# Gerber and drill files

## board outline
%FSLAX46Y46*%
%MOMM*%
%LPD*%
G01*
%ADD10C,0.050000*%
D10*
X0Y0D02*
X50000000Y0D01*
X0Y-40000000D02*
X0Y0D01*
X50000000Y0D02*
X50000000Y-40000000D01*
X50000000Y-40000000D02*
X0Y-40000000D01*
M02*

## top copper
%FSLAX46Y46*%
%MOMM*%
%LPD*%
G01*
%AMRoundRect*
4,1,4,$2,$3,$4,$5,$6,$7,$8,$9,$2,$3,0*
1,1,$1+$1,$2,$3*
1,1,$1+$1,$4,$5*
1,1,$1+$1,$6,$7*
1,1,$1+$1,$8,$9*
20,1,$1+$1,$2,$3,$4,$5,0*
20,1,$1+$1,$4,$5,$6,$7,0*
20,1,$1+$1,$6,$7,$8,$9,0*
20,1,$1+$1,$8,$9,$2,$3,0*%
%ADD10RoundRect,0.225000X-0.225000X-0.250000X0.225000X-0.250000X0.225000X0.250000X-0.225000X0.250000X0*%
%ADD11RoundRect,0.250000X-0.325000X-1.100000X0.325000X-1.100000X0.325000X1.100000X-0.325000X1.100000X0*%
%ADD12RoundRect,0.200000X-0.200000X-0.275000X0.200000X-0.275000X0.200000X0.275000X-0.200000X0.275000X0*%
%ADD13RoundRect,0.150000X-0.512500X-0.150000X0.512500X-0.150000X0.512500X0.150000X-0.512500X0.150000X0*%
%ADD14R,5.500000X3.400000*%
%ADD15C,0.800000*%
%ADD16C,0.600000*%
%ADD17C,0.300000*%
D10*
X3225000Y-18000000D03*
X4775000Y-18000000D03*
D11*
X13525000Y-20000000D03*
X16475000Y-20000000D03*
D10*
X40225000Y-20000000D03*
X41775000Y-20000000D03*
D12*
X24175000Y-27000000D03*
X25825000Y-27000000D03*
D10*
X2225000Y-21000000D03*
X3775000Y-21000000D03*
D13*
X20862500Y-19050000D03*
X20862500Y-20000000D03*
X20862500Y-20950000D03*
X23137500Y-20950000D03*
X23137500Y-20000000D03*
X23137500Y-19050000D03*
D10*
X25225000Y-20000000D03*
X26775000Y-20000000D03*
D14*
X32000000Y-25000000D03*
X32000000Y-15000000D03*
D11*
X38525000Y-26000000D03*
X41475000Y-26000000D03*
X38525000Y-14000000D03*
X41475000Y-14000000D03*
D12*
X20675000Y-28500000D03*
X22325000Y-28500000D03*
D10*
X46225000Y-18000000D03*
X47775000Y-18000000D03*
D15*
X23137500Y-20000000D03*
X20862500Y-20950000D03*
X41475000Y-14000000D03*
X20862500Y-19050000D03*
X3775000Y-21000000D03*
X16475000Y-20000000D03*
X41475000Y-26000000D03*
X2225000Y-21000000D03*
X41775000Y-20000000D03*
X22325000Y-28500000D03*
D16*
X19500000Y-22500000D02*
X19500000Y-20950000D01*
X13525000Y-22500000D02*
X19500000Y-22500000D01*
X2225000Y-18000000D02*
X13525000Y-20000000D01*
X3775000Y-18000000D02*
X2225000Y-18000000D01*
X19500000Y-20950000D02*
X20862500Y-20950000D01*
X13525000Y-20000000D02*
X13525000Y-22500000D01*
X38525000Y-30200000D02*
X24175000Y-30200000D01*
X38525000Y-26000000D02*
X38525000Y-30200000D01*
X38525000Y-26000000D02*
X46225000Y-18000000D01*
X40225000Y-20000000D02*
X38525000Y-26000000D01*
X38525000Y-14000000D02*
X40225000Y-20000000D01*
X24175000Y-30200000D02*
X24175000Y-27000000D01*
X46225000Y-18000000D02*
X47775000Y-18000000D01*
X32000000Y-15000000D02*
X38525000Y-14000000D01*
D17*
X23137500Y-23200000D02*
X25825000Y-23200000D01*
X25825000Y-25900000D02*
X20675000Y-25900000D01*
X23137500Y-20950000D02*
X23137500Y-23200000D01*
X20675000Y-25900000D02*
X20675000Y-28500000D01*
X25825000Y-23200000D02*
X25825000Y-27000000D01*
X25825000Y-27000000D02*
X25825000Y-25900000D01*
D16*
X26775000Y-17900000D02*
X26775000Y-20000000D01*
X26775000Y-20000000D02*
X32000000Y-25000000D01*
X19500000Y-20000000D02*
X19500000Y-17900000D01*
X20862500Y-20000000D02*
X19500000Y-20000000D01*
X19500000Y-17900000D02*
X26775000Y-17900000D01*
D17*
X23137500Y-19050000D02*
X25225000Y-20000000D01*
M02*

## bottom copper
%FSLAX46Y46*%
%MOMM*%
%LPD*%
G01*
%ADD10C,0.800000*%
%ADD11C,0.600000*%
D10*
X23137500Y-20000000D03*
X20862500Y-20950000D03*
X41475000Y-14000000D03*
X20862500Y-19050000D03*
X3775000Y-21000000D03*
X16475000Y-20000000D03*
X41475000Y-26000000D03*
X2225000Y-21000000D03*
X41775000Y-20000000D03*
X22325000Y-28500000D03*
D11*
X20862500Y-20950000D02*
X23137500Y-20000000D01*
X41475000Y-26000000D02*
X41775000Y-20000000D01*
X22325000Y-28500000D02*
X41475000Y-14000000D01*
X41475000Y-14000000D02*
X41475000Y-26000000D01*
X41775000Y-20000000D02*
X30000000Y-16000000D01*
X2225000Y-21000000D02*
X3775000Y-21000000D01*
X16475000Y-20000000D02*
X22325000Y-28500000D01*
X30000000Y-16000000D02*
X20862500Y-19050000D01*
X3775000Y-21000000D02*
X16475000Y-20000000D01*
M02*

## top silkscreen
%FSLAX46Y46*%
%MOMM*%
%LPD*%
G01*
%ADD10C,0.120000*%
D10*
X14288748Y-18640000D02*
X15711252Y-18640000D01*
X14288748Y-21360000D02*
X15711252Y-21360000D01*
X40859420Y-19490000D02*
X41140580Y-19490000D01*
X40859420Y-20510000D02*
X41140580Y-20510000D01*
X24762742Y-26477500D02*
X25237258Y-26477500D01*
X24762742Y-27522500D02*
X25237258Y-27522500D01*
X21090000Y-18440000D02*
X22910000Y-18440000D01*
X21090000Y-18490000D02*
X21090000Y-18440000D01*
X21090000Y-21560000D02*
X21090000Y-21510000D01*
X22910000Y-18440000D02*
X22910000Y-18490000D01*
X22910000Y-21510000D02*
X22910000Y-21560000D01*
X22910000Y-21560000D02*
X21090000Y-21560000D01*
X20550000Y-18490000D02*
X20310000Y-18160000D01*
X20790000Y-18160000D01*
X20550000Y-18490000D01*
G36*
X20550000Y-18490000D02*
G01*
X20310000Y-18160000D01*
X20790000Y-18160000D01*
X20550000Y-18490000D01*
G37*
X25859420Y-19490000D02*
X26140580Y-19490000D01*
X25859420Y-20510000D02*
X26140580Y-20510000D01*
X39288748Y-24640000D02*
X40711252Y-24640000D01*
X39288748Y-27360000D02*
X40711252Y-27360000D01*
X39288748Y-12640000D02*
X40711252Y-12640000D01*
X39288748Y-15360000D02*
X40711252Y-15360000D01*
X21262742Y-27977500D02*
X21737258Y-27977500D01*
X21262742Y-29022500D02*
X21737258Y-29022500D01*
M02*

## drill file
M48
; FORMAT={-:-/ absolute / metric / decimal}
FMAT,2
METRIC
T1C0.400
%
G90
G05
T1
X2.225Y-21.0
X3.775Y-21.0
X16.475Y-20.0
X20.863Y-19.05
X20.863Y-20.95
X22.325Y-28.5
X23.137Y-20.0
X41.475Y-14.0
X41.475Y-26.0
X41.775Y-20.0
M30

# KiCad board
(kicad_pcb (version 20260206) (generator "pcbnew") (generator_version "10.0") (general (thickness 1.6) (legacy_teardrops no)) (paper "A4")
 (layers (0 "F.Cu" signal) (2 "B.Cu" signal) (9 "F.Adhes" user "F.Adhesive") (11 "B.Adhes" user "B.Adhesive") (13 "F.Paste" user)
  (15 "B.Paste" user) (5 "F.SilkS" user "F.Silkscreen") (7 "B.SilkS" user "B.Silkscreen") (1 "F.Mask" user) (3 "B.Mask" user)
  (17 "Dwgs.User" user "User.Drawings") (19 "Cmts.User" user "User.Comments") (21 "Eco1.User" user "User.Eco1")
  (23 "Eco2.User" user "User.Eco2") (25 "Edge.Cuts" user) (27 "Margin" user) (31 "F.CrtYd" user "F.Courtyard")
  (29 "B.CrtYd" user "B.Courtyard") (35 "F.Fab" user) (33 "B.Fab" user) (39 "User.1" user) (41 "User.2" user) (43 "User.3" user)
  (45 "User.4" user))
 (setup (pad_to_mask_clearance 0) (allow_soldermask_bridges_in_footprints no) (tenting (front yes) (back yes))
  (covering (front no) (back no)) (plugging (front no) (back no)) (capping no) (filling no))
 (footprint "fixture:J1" (layer "F.Cu") (at 4 18)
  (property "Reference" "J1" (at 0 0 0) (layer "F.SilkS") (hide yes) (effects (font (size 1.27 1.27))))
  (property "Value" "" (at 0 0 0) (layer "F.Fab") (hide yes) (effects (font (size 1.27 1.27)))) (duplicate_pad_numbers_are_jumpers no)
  (pad "1" smd roundrect (at -0.775 0) (size 0.9 0.95) (layers "F.Cu" "F.Mask" "F.Paste") (roundrect_rratio 0.25) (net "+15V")
   (thermal_bridge_angle 45))
  (pad "2" smd roundrect (at 0.775 0) (size 0.9 0.95) (layers "F.Cu" "F.Mask" "F.Paste") (roundrect_rratio 0.25) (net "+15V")
   (thermal_bridge_angle 45)))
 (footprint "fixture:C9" (layer "F.Cu") (at 15 20)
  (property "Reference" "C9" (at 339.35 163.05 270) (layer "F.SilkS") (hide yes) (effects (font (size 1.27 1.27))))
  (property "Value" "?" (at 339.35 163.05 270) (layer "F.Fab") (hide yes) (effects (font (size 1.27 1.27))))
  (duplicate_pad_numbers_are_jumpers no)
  (fp_line (start -0.711252 -1.36) (end 0.711252 -1.36) (stroke (width 0.12) (type solid)) (layer "F.SilkS"))
  (fp_line (start -0.711252 1.36) (end 0.711252 1.36) (stroke (width 0.12) (type solid)) (layer "F.SilkS"))
  (pad "1" smd roundrect (at -1.475 0) (size 1.15 2.7) (layers "F.Cu" "F.Mask" "F.Paste") (roundrect_rratio 0.217391) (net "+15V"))
  (pad "2" smd roundrect (at 1.475 0) (size 1.15 2.7) (layers "F.Cu" "F.Mask" "F.Paste") (roundrect_rratio 0.217391) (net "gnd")))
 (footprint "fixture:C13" (layer "F.Cu") (at 41 20)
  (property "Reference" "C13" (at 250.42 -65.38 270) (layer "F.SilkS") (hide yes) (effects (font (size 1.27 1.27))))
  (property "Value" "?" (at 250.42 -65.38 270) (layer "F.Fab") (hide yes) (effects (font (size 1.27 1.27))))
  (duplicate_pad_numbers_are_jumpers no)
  (fp_line (start -0.14058 -0.51) (end 0.14058 -0.51) (stroke (width 0.12) (type solid)) (layer "F.SilkS"))
  (fp_line (start -0.14058 0.51) (end 0.14058 0.51) (stroke (width 0.12) (type solid)) (layer "F.SilkS"))
  (pad "1" smd roundrect (at -0.775 0) (size 0.9 0.95) (layers "F.Cu" "F.Mask" "F.Paste") (roundrect_rratio 0.25) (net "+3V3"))
  (pad "2" smd roundrect (at 0.775 0) (size 0.9 0.95) (layers "F.Cu" "F.Mask" "F.Paste") (roundrect_rratio 0.25) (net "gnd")))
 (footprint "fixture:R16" (layer "F.Cu") (at 25 27)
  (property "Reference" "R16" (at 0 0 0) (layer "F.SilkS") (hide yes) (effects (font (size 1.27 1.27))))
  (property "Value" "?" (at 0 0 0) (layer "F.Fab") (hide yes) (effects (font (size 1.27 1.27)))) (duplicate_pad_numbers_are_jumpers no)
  (fp_line (start -0.237258 -0.5225) (end 0.237258 -0.5225) (stroke (width 0.12) (type solid)) (layer "F.SilkS"))
  (fp_line (start -0.237258 0.5225) (end 0.237258 0.5225) (stroke (width 0.12) (type solid)) (layer "F.SilkS"))
  (pad "1" smd roundrect (at -0.825 0) (size 0.8 0.95) (layers "F.Cu" "F.Mask" "F.Paste") (roundrect_rratio 0.25) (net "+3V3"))
  (pad "2" smd roundrect (at 0.825 0) (size 0.8 0.95) (layers "F.Cu" "F.Mask" "F.Paste") (roundrect_rratio 0.25) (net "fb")))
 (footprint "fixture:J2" (layer "F.Cu") (at 3 21)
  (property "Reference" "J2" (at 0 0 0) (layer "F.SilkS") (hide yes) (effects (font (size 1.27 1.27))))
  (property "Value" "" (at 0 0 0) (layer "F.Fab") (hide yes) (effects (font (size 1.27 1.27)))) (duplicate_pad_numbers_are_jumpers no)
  (pad "1" smd roundrect (at -0.775 0) (size 0.9 0.95) (layers "F.Cu" "F.Mask" "F.Paste") (roundrect_rratio 0.25) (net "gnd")
   (thermal_bridge_angle 45))
  (pad "2" smd roundrect (at 0.775 0) (size 0.9 0.95) (layers "F.Cu" "F.Mask" "F.Paste") (roundrect_rratio 0.25) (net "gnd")
   (thermal_bridge_angle 45)))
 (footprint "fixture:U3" (layer "F.Cu") (at 22 20)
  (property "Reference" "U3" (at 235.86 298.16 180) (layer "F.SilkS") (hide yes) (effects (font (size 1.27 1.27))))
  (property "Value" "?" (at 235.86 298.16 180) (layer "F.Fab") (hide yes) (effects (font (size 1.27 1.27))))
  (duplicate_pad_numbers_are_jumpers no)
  (fp_line (start -0.91 -1.56) (end 0.91 -1.56) (stroke (width 0.12) (type solid)) (layer "F.SilkS"))
  (fp_line (start -0.91 -1.51) (end -0.91 -1.56) (stroke (width 0.12) (type solid)) (layer "F.SilkS"))
  (fp_line (start -0.91 1.56) (end -0.91 1.51) (stroke (width 0.12) (type solid)) (layer "F.SilkS"))
  (fp_line (start 0.91 -1.56) (end 0.91 -1.51) (stroke (width 0.12) (type solid)) (layer "F.SilkS"))
  (fp_line (start 0.91 1.51) (end 0.91 1.56) (stroke (width 0.12) (type solid)) (layer "F.SilkS"))
  (fp_line (start 0.91 1.56) (end -0.91 1.56) (stroke (width 0.12) (type solid)) (layer "F.SilkS"))
  (fp_poly (pts (xy -1.45 -1.51) (xy -1.69 -1.84) (xy -1.21 -1.84)) (stroke (width 0.12) (type solid)) (fill yes) (layer "F.SilkS"))
  (pad "1" smd roundrect (at -1.1375 -0.95) (size 1.325 0.6) (layers "F.Cu" "F.Mask" "F.Paste") (roundrect_rratio 0.25) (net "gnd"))
  (pad "2" smd roundrect (at -1.1375 0) (size 1.325 0.6) (layers "F.Cu" "F.Mask" "F.Paste") (roundrect_rratio 0.25) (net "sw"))
  (pad "3" smd roundrect (at -1.1375 0.95) (size 1.325 0.6) (layers "F.Cu" "F.Mask" "F.Paste") (roundrect_rratio 0.25) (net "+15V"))
  (pad "4" smd roundrect (at 1.1375 0.95) (size 1.325 0.6) (layers "F.Cu" "F.Mask" "F.Paste") (roundrect_rratio 0.25) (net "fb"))
  (pad "5" smd roundrect (at 1.1375 0) (size 1.325 0.6) (layers "F.Cu" "F.Mask" "F.Paste") (roundrect_rratio 0.25) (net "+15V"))
  (pad "6" smd roundrect (at 1.1375 -0.95) (size 1.325 0.6) (layers "F.Cu" "F.Mask" "F.Paste") (roundrect_rratio 0.25) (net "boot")))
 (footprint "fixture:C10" (layer "F.Cu") (at 26 20)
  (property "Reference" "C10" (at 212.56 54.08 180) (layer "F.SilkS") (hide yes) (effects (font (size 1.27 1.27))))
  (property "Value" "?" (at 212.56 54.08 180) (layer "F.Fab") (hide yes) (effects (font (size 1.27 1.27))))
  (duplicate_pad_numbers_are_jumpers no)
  (fp_line (start -0.14058 -0.51) (end 0.14058 -0.51) (stroke (width 0.12) (type solid)) (layer "F.SilkS"))
  (fp_line (start -0.14058 0.51) (end 0.14058 0.51) (stroke (width 0.12) (type solid)) (layer "F.SilkS"))
  (pad "1" smd roundrect (at -0.775 0) (size 0.9 0.95) (layers "F.Cu" "F.Mask" "F.Paste") (roundrect_rratio 0.25) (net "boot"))
  (pad "2" smd roundrect (at 0.775 0) (size 0.9 0.95) (layers "F.Cu" "F.Mask" "F.Paste") (roundrect_rratio 0.25) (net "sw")))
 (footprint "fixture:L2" (layer "F.Cu") (at 32 20 90)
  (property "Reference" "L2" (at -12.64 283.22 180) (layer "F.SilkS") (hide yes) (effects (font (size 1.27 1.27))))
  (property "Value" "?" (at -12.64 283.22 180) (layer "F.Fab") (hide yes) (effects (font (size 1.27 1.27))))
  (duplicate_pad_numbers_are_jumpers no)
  (pad "1" smd rect (at -5 0 90) (size 3.4 5.5) (layers "F.Cu" "F.Mask" "F.Paste") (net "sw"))
  (pad "2" smd rect (at 5 0 90) (size 3.4 5.5) (layers "F.Cu" "F.Mask" "F.Paste") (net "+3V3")))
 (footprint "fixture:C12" (layer "F.Cu") (at 40 26)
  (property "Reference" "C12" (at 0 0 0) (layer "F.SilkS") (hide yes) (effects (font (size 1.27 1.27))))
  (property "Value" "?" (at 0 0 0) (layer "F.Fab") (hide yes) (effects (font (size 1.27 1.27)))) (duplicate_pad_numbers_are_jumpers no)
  (fp_line (start -0.711252 -1.36) (end 0.711252 -1.36) (stroke (width 0.12) (type solid)) (layer "F.SilkS"))
  (fp_line (start -0.711252 1.36) (end 0.711252 1.36) (stroke (width 0.12) (type solid)) (layer "F.SilkS"))
  (pad "1" smd roundrect (at -1.475 0) (size 1.15 2.7) (layers "F.Cu" "F.Mask" "F.Paste") (roundrect_rratio 0.217391) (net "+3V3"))
  (pad "2" smd roundrect (at 1.475 0) (size 1.15 2.7) (layers "F.Cu" "F.Mask" "F.Paste") (roundrect_rratio 0.217391) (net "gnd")))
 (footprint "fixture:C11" (layer "F.Cu") (at 40 14)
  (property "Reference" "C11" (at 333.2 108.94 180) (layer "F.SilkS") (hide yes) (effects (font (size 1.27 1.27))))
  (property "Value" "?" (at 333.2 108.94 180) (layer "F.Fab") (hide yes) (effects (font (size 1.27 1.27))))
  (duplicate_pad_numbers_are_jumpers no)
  (fp_line (start -0.711252 -1.36) (end 0.711252 -1.36) (stroke (width 0.12) (type solid)) (layer "F.SilkS"))
  (fp_line (start -0.711252 1.36) (end 0.711252 1.36) (stroke (width 0.12) (type solid)) (layer "F.SilkS"))
  (pad "1" smd roundrect (at -1.475 0) (size 1.15 2.7) (layers "F.Cu" "F.Mask" "F.Paste") (roundrect_rratio 0.217391) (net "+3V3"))
  (pad "2" smd roundrect (at 1.475 0) (size 1.15 2.7) (layers "F.Cu" "F.Mask" "F.Paste") (roundrect_rratio 0.217391) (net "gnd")))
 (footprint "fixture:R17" (layer "F.Cu") (at 21.5 28.5)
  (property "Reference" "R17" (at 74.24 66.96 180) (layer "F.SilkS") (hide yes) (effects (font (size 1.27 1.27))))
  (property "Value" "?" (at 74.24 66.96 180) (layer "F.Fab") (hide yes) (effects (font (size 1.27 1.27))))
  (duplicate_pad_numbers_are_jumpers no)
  (fp_line (start -0.237258 -0.5225) (end 0.237258 -0.5225) (stroke (width 0.12) (type solid)) (layer "F.SilkS"))
  (fp_line (start -0.237258 0.5225) (end 0.237258 0.5225) (stroke (width 0.12) (type solid)) (layer "F.SilkS"))
  (pad "1" smd roundrect (at -0.825 0) (size 0.8 0.95) (layers "F.Cu" "F.Mask" "F.Paste") (roundrect_rratio 0.25) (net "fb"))
  (pad "2" smd roundrect (at 0.825 0) (size 0.8 0.95) (layers "F.Cu" "F.Mask" "F.Paste") (roundrect_rratio 0.25) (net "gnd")))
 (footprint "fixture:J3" (layer "F.Cu") (at 47 18)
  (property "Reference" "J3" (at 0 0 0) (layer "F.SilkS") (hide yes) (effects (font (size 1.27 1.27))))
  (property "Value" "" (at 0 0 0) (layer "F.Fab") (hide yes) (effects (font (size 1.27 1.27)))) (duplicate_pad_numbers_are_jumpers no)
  (pad "1" smd roundrect (at -0.775 0) (size 0.9 0.95) (layers "F.Cu" "F.Mask" "F.Paste") (roundrect_rratio 0.25) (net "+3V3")
   (thermal_bridge_angle 45))
  (pad "2" smd roundrect (at 0.775 0) (size 0.9 0.95) (layers "F.Cu" "F.Mask" "F.Paste") (roundrect_rratio 0.25) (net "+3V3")
   (thermal_bridge_angle 45)))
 (gr_line (start 0 0) (end 50 0) (stroke (width 0.05) (type default)) (layer "Edge.Cuts"))
 (gr_line (start 0 40) (end 0 0) (stroke (width 0.05) (type default)) (layer "Edge.Cuts"))
 (gr_line (start 50 0) (end 50 40) (stroke (width 0.05) (type default)) (layer "Edge.Cuts"))
 (gr_line (start 50 40) (end 0 40) (stroke (width 0.05) (type default)) (layer "Edge.Cuts"))
 (segment (start 19.5 22.5) (end 19.5 20.95) (width 0.6) (layer "F.Cu") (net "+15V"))
 (segment (start 13.525 22.5) (end 19.5 22.5) (width 0.6) (layer "F.Cu") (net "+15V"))
 (segment (start 2.225 18) (end 13.525 20) (width 0.6) (layer "F.Cu") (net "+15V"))
 (segment (start 3.775 18) (end 2.225 18) (width 0.6) (layer "F.Cu") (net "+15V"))
 (segment (start 19.5 20.95) (end 20.8625 20.95) (width 0.6) (layer "F.Cu") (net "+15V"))
 (segment (start 13.525 20) (end 13.525 22.5) (width 0.6) (layer "F.Cu") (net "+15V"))
 (via (at 23.1375 20) (size 0.8) (drill 0.4) (layers "F.Cu" "B.Cu") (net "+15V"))
 (via (at 20.8625 20.95) (size 0.8) (drill 0.4) (layers "F.Cu" "B.Cu") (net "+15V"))
 (segment (start 20.8625 20.95) (end 23.1375 20) (width 0.6) (layer "B.Cu") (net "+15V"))
 (via (at 41.475 14) (size 0.8) (drill 0.4) (layers "F.Cu" "B.Cu") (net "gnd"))
 (via (at 20.8625 19.05) (size 0.8) (drill 0.4) (layers "F.Cu" "B.Cu") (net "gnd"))
 (via (at 3.775 21) (size 0.8) (drill 0.4) (layers "F.Cu" "B.Cu") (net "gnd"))
 (via (at 16.475 20) (size 0.8) (drill 0.4) (layers "F.Cu" "B.Cu") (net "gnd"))
 (via (at 41.475 26) (size 0.8) (drill 0.4) (layers "F.Cu" "B.Cu") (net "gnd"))
 (via (at 2.225 21) (size 0.8) (drill 0.4) (layers "F.Cu" "B.Cu") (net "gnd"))
 (via (at 41.775 20) (size 0.8) (drill 0.4) (layers "F.Cu" "B.Cu") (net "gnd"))
 (via (at 22.325 28.5) (size 0.8) (drill 0.4) (layers "F.Cu" "B.Cu") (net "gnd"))
 (segment (start 41.475 26) (end 41.775 20) (width 0.6) (layer "B.Cu") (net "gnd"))
 (segment (start 22.325 28.5) (end 41.475 14) (width 0.6) (layer "B.Cu") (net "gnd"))
 (segment (start 41.475 14) (end 41.475 26) (width 0.6) (layer "B.Cu") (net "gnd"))
 (segment (start 41.775 20) (end 30 16) (width 0.6) (layer "B.Cu") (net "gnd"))
 (segment (start 2.225 21) (end 3.775 21) (width 0.6) (layer "B.Cu") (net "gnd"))
 (segment (start 16.475 20) (end 22.325 28.5) (width 0.6) (layer "B.Cu") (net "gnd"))
 (segment (start 30 16) (end 20.8625 19.05) (width 0.6) (layer "B.Cu") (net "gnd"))
 (segment (start 3.775 21) (end 16.475 20) (width 0.6) (layer "B.Cu") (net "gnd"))
 (segment (start 38.525 30.2) (end 24.175 30.2) (width 0.6) (layer "F.Cu") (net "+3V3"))
 (segment (start 38.525 26) (end 38.525 30.2) (width 0.6) (layer "F.Cu") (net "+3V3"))
 (segment (start 38.525 26) (end 46.225 18) (width 0.6) (layer "F.Cu") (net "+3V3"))
 (segment (start 40.225 20) (end 38.525 26) (width 0.6) (layer "F.Cu") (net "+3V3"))
 (segment (start 38.525 14) (end 40.225 20) (width 0.6) (layer "F.Cu") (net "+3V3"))
 (segment (start 24.175 30.2) (end 24.175 27) (width 0.6) (layer "F.Cu") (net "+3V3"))
 (segment (start 46.225 18) (end 47.775 18) (width 0.6) (layer "F.Cu") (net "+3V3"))
 (segment (start 32 15) (end 38.525 14) (width 0.6) (layer "F.Cu") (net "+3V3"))
 (segment (start 23.1375 23.2) (end 25.825 23.2) (width 0.3) (layer "F.Cu") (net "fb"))
 (segment (start 25.825 25.9) (end 20.675 25.9) (width 0.3) (layer "F.Cu") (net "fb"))
 (segment (start 23.1375 20.95) (end 23.1375 23.2) (width 0.3) (layer "F.Cu") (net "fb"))
 (segment (start 20.675 25.9) (end 20.675 28.5) (width 0.3) (layer "F.Cu") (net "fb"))
 (segment (start 25.825 23.2) (end 25.825 27) (width 0.3) (layer "F.Cu") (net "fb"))
 (segment (start 25.825 27) (end 25.825 25.9) (width 0.3) (layer "F.Cu") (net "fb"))
 (segment (start 26.775 17.9) (end 26.775 20) (width 0.6) (layer "F.Cu") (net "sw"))
 (segment (start 26.775 20) (end 32 25) (width 0.6) (layer "F.Cu") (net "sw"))
 (segment (start 19.5 20) (end 19.5 17.9) (width 0.6) (layer "F.Cu") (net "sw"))
 (segment (start 20.8625 20) (end 19.5 20) (width 0.6) (layer "F.Cu") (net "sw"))
 (segment (start 19.5 17.9) (end 26.775 17.9) (width 0.6) (layer "F.Cu") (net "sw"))
 (segment (start 23.1375 19.05) (end 25.225 20) (width 0.3) (layer "F.Cu") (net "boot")))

